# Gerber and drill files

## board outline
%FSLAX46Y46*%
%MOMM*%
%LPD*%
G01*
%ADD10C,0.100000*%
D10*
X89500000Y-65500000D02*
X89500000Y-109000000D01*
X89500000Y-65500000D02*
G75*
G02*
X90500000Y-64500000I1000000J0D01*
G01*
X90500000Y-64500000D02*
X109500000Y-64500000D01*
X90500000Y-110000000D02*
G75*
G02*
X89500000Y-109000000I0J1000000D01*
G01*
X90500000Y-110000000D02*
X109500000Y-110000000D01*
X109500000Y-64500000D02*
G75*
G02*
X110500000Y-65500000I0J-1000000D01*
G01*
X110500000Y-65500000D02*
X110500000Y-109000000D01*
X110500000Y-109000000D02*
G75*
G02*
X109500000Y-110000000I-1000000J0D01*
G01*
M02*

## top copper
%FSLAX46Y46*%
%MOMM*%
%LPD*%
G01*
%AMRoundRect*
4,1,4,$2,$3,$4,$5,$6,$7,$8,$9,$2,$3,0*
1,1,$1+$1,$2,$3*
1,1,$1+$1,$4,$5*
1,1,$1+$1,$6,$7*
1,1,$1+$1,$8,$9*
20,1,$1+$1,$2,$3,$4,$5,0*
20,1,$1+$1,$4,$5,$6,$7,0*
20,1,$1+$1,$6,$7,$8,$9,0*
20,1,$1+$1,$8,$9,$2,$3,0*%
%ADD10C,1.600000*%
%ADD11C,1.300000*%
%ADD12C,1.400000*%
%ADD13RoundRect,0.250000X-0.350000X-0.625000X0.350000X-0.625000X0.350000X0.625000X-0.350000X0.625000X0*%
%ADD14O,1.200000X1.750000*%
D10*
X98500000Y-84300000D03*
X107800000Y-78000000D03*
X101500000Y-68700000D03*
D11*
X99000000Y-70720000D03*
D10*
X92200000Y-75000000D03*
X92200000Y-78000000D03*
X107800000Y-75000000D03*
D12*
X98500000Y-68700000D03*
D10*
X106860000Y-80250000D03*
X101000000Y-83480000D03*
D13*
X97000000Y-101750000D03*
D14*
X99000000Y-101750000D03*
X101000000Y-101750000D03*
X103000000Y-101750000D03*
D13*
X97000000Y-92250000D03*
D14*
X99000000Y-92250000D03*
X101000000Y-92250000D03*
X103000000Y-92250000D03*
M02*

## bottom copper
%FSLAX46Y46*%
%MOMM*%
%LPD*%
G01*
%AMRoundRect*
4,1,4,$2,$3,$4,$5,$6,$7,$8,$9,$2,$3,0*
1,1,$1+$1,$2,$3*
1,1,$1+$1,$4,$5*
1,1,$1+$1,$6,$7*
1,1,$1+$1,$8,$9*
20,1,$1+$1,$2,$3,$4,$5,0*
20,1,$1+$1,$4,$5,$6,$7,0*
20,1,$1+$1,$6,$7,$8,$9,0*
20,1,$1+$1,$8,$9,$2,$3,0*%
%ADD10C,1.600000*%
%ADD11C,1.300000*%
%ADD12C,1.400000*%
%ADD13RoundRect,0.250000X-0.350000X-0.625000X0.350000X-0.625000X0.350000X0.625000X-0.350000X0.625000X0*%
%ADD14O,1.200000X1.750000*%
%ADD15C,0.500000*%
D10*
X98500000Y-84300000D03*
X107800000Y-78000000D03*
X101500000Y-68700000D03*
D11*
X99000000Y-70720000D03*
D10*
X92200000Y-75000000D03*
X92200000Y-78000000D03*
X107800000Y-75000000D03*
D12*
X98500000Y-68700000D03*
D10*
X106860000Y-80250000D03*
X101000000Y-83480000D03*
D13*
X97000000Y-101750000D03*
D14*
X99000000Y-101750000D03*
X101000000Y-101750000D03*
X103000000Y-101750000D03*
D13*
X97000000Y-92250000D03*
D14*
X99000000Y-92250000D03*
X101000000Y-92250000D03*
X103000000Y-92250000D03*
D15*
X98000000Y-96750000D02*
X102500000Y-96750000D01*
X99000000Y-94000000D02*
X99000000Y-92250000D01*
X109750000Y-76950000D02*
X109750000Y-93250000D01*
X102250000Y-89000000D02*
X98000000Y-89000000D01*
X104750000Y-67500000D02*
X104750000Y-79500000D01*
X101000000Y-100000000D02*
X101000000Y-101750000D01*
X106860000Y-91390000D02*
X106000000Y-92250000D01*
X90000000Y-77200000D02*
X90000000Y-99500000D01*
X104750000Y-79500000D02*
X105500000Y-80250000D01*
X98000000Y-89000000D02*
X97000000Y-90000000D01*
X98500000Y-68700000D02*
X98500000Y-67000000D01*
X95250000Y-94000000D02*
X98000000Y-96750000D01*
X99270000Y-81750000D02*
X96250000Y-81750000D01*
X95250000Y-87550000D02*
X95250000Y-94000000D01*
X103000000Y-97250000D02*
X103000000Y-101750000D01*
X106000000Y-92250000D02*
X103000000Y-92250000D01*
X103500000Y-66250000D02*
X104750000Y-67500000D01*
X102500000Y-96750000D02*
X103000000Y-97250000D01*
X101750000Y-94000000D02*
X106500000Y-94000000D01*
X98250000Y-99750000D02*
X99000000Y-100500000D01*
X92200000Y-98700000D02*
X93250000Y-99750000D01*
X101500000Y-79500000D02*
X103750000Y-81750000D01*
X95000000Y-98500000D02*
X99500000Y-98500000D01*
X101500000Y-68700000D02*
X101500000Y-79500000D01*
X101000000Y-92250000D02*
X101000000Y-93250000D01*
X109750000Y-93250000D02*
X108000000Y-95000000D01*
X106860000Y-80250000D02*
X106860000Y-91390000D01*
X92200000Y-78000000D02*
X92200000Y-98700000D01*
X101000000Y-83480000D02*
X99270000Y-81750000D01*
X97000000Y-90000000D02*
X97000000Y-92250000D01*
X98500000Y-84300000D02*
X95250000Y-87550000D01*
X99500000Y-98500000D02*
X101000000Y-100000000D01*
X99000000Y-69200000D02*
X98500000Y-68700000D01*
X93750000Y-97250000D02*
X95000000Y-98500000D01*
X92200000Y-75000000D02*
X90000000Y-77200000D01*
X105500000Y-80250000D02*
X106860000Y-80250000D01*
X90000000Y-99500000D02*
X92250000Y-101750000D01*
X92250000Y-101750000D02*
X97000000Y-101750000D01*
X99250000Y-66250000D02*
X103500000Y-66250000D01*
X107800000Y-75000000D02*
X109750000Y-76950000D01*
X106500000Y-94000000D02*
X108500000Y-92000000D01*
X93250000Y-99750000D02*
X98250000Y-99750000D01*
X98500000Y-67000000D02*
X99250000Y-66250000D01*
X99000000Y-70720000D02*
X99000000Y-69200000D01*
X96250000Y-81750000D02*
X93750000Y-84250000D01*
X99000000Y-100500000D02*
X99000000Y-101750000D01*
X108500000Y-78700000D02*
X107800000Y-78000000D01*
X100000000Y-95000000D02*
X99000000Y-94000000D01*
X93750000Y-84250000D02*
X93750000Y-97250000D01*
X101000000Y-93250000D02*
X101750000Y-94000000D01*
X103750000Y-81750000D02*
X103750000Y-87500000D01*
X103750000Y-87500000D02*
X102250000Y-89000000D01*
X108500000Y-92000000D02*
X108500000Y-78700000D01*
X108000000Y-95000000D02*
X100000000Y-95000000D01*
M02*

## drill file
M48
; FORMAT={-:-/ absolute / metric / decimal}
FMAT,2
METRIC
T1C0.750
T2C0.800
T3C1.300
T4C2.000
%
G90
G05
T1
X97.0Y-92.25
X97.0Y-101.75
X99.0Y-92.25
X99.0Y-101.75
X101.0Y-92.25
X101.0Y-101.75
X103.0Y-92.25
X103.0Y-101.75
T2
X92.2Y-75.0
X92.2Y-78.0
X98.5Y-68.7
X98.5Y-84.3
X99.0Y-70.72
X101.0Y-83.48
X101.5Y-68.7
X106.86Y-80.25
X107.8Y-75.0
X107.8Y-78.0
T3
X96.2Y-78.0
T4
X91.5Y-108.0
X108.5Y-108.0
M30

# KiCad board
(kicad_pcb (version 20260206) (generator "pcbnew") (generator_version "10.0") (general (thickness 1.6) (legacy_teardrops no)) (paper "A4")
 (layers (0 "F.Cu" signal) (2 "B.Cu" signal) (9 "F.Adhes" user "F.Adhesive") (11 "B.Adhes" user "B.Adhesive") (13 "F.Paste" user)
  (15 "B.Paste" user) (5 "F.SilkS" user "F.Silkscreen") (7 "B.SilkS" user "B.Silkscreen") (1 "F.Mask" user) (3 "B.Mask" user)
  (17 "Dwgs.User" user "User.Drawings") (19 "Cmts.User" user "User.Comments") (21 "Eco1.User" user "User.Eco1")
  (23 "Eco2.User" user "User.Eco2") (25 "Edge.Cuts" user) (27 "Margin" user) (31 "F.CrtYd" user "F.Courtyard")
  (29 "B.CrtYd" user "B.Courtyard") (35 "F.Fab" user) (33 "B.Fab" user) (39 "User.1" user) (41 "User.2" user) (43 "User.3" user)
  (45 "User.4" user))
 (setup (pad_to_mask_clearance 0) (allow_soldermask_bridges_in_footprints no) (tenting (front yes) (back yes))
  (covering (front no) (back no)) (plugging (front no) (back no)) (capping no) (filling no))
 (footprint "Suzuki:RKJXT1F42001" (layer "F.Cu") (at 100 76.5)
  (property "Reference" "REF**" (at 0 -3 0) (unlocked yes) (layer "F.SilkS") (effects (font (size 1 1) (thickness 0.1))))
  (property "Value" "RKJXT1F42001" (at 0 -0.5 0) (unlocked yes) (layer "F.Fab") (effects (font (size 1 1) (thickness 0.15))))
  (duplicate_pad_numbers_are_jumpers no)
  (pad "" np_thru_hole circle (at -3.8 1.5) (size 1.3 1.3) (drill 1.3) (layers "*.Cu" "*.Mask"))
  (pad "A" thru_hole circle (at -1.5 7.8) (size 1.6 1.6) (drill 0.8) (layers "*.Cu" "*.Mask") (remove_unused_layers no))
  (pad "B" thru_hole circle (at 7.8 1.5) (size 1.6 1.6) (drill 0.8) (layers "*.Cu" "*.Mask") (remove_unused_layers no))
  (pad "C" thru_hole circle (at 1.5 -7.8) (size 1.6 1.6) (drill 0.8) (layers "*.Cu" "*.Mask") (remove_unused_layers no))
  (pad "Com" thru_hole circle (at -1 -5.78) (size 1.3 1.3) (drill 0.8) (layers "*.Cu" "*.Mask") (remove_unused_layers no))
  (pad "D" thru_hole circle (at -7.8 -1.5) (size 1.6 1.6) (drill 0.8) (layers "*.Cu" "*.Mask") (remove_unused_layers no))
  (pad "EA" thru_hole circle (at -7.8 1.5) (size 1.6 1.6) (drill 0.8) (layers "*.Cu" "*.Mask") (remove_unused_layers no))
  (pad "EB" thru_hole circle (at 7.8 -1.5) (size 1.6 1.6) (drill 0.8) (layers "*.Cu" "*.Mask") (remove_unused_layers no))
  (pad "ECom" thru_hole circle (at -1.5 -7.8) (size 1.4 1.4) (drill 0.8) (layers "*.Cu" "*.Mask") (remove_unused_layers no))
  (pad "GND" thru_hole circle (at 6.86 3.75) (size 1.6 1.6) (drill 0.8) (layers "*.Cu" "*.Mask") (remove_unused_layers no))
  (pad "Push" thru_hole circle (at 1 6.98) (size 1.6 1.6) (drill 0.8) (layers "*.Cu" "*.Mask") (remove_unused_layers no)))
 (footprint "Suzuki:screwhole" (layer "F.Cu") (at 108.75 108)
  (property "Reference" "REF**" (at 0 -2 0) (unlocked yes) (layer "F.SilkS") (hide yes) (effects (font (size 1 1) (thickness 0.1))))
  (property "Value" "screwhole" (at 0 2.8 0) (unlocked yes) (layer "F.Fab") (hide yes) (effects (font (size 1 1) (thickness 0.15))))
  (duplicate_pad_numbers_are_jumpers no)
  (pad "" np_thru_hole circle (at -0.25 0) (size 2 2) (drill 2) (layers "*.Cu" "*.Mask")))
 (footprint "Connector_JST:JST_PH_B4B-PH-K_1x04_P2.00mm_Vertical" (layer "F.Cu") (at 97 101.75)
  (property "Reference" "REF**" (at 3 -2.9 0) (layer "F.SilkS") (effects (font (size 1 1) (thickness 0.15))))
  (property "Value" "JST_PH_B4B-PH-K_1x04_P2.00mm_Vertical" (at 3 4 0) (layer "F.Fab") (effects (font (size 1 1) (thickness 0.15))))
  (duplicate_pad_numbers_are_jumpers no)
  (pad "1" thru_hole roundrect (at 0 0) (size 1.2 1.75) (drill 0.75) (layers "*.Cu" "*.Mask") (remove_unused_layers no)
   (roundrect_rratio 0.208333))
  (pad "2" thru_hole oval (at 2 0) (size 1.2 1.75) (drill 0.75) (layers "*.Cu" "*.Mask") (remove_unused_layers no))
  (pad "3" thru_hole oval (at 4 0) (size 1.2 1.75) (drill 0.75) (layers "*.Cu" "*.Mask") (remove_unused_layers no))
  (pad "4" thru_hole oval (at 6 0) (size 1.2 1.75) (drill 0.75) (layers "*.Cu" "*.Mask") (remove_unused_layers no)))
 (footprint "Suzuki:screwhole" (layer "F.Cu") (at 91.5 108)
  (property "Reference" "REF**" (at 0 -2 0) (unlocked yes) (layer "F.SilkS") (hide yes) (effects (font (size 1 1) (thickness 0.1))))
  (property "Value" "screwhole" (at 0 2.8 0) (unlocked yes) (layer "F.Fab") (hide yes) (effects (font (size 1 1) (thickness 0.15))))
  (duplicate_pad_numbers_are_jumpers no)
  (pad "" np_thru_hole circle (at 0 0) (size 2 2) (drill 2) (layers "*.Cu" "*.Mask")))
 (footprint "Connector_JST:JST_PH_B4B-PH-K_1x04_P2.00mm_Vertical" (layer "F.Cu") (at 97 92.25)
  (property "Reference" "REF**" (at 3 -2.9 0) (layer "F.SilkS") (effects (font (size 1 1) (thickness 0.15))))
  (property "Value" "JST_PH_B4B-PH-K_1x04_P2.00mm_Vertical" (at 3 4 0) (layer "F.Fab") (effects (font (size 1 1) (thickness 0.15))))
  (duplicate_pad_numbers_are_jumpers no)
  (pad "1" thru_hole roundrect (at 0 0) (size 1.2 1.75) (drill 0.75) (layers "*.Cu" "*.Mask") (remove_unused_layers no)
   (roundrect_rratio 0.208333))
  (pad "2" thru_hole oval (at 2 0) (size 1.2 1.75) (drill 0.75) (layers "*.Cu" "*.Mask") (remove_unused_layers no))
  (pad "3" thru_hole oval (at 4 0) (size 1.2 1.75) (drill 0.75) (layers "*.Cu" "*.Mask") (remove_unused_layers no))
  (pad "4" thru_hole oval (at 6 0) (size 1.2 1.75) (drill 0.75) (layers "*.Cu" "*.Mask") (remove_unused_layers no)))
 (gr_line (start 89.5 65.5) (end 89.5 109) (stroke (width 0.1) (type solid)) (layer "Edge.Cuts"))
 (gr_arc (start 89.5 65.5) (mid 89.792893 64.792893) (end 90.5 64.5) (stroke (width 0.1) (type default)) (layer "Edge.Cuts"))
 (gr_line (start 90.5 64.5) (end 109.5 64.5) (stroke (width 0.1) (type solid)) (layer "Edge.Cuts"))
 (gr_arc (start 90.5 110) (mid 89.792893 109.707107) (end 89.5 109) (stroke (width 0.1) (type default)) (layer "Edge.Cuts"))
 (gr_line (start 90.5 110) (end 109.5 110) (stroke (width 0.1) (type solid)) (layer "Edge.Cuts"))
 (gr_arc (start 109.5 64.5) (mid 110.207107 64.792893) (end 110.5 65.5) (stroke (width 0.1) (type default)) (layer "Edge.Cuts"))
 (gr_line (start 110.5 65.5) (end 110.5 109) (stroke (width 0.1) (type solid)) (layer "Edge.Cuts"))
 (gr_arc (start 110.5 109) (mid 110.207107 109.707107) (end 109.5 110) (stroke (width 0.1) (type default)) (layer "Edge.Cuts"))
 (segment (start 98 96.75) (end 102.5 96.75) (width 0.5) (layer "B.Cu") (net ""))
 (segment (start 99 94) (end 99 92.25) (width 0.5) (layer "B.Cu") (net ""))
 (segment (start 109.75 76.95) (end 109.75 93.25) (width 0.5) (layer "B.Cu") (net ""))
 (segment (start 102.25 89) (end 98 89) (width 0.5) (layer "B.Cu") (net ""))
 (segment (start 104.75 67.5) (end 104.75 79.5) (width 0.5) (layer "B.Cu") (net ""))
 (segment (start 101 100) (end 101 101.75) (width 0.5) (layer "B.Cu") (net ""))
 (segment (start 106.86 91.39) (end 106 92.25) (width 0.5) (layer "B.Cu") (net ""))
 (segment (start 90 77.2) (end 90 99.5) (width 0.5) (layer "B.Cu") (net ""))
 (segment (start 104.75 79.5) (end 105.5 80.25) (width 0.5) (layer "B.Cu") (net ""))
 (segment (start 98 89) (end 97 90) (width 0.5) (layer "B.Cu") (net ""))
 (segment (start 98.5 68.7) (end 98.5 67) (width 0.5) (layer "B.Cu") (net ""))
 (segment (start 95.25 94) (end 98 96.75) (width 0.5) (layer "B.Cu") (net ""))
 (segment (start 99.27 81.75) (end 96.25 81.75) (width 0.5) (layer "B.Cu") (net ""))
 (segment (start 95.25 87.55) (end 95.25 94) (width 0.5) (layer "B.Cu") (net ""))
 (segment (start 103 97.25) (end 103 101.75) (width 0.5) (layer "B.Cu") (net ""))
 (segment (start 106 92.25) (end 103 92.25) (width 0.5) (layer "B.Cu") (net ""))
 (segment (start 103.5 66.25) (end 104.75 67.5) (width 0.5) (layer "B.Cu") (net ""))
 (segment (start 102.5 96.75) (end 103 97.25) (width 0.5) (layer "B.Cu") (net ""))
 (segment (start 101.75 94) (end 106.5 94) (width 0.5) (layer "B.Cu") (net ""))
 (segment (start 98.25 99.75) (end 99 100.5) (width 0.5) (layer "B.Cu") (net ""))
 (segment (start 92.2 98.7) (end 93.25 99.75) (width 0.5) (layer "B.Cu") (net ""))
 (segment (start 101.5 79.5) (end 103.75 81.75) (width 0.5) (layer "B.Cu") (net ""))
 (segment (start 95 98.5) (end 99.5 98.5) (width 0.5) (layer "B.Cu") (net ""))
 (segment (start 101.5 68.7) (end 101.5 79.5) (width 0.5) (layer "B.Cu") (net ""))
 (segment (start 101 92.25) (end 101 93.25) (width 0.5) (layer "B.Cu") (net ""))
 (segment (start 109.75 93.25) (end 108 95) (width 0.5) (layer "B.Cu") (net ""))
 (segment (start 106.86 80.25) (end 106.86 91.39) (width 0.5) (layer "B.Cu") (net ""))
 (segment (start 92.2 78) (end 92.2 98.7) (width 0.5) (layer "B.Cu") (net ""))
 (segment (start 101 83.48) (end 99.27 81.75) (width 0.5) (layer "B.Cu") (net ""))
 (segment (start 97 90) (end 97 92.25) (width 0.5) (layer "B.Cu") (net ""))
 (segment (start 98.5 84.3) (end 95.25 87.55) (width 0.5) (layer "B.Cu") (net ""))
 (segment (start 99.5 98.5) (end 101 100) (width 0.5) (layer "B.Cu") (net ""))
 (segment (start 99 69.2) (end 98.5 68.7) (width 0.5) (layer "B.Cu") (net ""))
 (segment (start 93.75 97.25) (end 95 98.5) (width 0.5) (layer "B.Cu") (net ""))
 (segment (start 92.2 75) (end 90 77.2) (width 0.5) (layer "B.Cu") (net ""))
 (segment (start 105.5 80.25) (end 106.86 80.25) (width 0.5) (layer "B.Cu") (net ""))
 (segment (start 90 99.5) (end 92.25 101.75) (width 0.5) (layer "B.Cu") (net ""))
 (segment (start 92.25 101.75) (end 97 101.75) (width 0.5) (layer "B.Cu") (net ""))
 (segment (start 99.25 66.25) (end 103.5 66.25) (width 0.5) (layer "B.Cu") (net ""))
 (segment (start 107.8 75) (end 109.75 76.95) (width 0.5) (layer "B.Cu") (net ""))
 (segment (start 106.5 94) (end 108.5 92) (width 0.5) (layer "B.Cu") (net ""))
 (segment (start 93.25 99.75) (end 98.25 99.75) (width 0.5) (layer "B.Cu") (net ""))
 (segment (start 98.5 67) (end 99.25 66.25) (width 0.5) (layer "B.Cu") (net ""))
 (segment (start 99 70.72) (end 99 69.2) (width 0.5) (layer "B.Cu") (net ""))
 (segment (start 96.25 81.75) (end 93.75 84.25) (width 0.5) (layer "B.Cu") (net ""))
 (segment (start 99 100.5) (end 99 101.75) (width 0.5) (layer "B.Cu") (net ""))
 (segment (start 108.5 78.7) (end 107.8 78) (width 0.5) (layer "B.Cu") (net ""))
 (segment (start 100 95) (end 99 94) (width 0.5) (layer "B.Cu") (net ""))
 (segment (start 93.75 84.25) (end 93.75 97.25) (width 0.5) (layer "B.Cu") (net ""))
 (segment (start 101 93.25) (end 101.75 94) (width 0.5) (layer "B.Cu") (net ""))
 (segment (start 103.75 81.75) (end 103.75 87.5) (width 0.5) (layer "B.Cu") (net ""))
 (segment (start 103.75 87.5) (end 102.25 89) (width 0.5) (layer "B.Cu") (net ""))
 (segment (start 108.5 92) (end 108.5 78.7) (width 0.5) (layer "B.Cu") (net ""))
 (segment (start 108 95) (end 100 95) (width 0.5) (layer "B.Cu") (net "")))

